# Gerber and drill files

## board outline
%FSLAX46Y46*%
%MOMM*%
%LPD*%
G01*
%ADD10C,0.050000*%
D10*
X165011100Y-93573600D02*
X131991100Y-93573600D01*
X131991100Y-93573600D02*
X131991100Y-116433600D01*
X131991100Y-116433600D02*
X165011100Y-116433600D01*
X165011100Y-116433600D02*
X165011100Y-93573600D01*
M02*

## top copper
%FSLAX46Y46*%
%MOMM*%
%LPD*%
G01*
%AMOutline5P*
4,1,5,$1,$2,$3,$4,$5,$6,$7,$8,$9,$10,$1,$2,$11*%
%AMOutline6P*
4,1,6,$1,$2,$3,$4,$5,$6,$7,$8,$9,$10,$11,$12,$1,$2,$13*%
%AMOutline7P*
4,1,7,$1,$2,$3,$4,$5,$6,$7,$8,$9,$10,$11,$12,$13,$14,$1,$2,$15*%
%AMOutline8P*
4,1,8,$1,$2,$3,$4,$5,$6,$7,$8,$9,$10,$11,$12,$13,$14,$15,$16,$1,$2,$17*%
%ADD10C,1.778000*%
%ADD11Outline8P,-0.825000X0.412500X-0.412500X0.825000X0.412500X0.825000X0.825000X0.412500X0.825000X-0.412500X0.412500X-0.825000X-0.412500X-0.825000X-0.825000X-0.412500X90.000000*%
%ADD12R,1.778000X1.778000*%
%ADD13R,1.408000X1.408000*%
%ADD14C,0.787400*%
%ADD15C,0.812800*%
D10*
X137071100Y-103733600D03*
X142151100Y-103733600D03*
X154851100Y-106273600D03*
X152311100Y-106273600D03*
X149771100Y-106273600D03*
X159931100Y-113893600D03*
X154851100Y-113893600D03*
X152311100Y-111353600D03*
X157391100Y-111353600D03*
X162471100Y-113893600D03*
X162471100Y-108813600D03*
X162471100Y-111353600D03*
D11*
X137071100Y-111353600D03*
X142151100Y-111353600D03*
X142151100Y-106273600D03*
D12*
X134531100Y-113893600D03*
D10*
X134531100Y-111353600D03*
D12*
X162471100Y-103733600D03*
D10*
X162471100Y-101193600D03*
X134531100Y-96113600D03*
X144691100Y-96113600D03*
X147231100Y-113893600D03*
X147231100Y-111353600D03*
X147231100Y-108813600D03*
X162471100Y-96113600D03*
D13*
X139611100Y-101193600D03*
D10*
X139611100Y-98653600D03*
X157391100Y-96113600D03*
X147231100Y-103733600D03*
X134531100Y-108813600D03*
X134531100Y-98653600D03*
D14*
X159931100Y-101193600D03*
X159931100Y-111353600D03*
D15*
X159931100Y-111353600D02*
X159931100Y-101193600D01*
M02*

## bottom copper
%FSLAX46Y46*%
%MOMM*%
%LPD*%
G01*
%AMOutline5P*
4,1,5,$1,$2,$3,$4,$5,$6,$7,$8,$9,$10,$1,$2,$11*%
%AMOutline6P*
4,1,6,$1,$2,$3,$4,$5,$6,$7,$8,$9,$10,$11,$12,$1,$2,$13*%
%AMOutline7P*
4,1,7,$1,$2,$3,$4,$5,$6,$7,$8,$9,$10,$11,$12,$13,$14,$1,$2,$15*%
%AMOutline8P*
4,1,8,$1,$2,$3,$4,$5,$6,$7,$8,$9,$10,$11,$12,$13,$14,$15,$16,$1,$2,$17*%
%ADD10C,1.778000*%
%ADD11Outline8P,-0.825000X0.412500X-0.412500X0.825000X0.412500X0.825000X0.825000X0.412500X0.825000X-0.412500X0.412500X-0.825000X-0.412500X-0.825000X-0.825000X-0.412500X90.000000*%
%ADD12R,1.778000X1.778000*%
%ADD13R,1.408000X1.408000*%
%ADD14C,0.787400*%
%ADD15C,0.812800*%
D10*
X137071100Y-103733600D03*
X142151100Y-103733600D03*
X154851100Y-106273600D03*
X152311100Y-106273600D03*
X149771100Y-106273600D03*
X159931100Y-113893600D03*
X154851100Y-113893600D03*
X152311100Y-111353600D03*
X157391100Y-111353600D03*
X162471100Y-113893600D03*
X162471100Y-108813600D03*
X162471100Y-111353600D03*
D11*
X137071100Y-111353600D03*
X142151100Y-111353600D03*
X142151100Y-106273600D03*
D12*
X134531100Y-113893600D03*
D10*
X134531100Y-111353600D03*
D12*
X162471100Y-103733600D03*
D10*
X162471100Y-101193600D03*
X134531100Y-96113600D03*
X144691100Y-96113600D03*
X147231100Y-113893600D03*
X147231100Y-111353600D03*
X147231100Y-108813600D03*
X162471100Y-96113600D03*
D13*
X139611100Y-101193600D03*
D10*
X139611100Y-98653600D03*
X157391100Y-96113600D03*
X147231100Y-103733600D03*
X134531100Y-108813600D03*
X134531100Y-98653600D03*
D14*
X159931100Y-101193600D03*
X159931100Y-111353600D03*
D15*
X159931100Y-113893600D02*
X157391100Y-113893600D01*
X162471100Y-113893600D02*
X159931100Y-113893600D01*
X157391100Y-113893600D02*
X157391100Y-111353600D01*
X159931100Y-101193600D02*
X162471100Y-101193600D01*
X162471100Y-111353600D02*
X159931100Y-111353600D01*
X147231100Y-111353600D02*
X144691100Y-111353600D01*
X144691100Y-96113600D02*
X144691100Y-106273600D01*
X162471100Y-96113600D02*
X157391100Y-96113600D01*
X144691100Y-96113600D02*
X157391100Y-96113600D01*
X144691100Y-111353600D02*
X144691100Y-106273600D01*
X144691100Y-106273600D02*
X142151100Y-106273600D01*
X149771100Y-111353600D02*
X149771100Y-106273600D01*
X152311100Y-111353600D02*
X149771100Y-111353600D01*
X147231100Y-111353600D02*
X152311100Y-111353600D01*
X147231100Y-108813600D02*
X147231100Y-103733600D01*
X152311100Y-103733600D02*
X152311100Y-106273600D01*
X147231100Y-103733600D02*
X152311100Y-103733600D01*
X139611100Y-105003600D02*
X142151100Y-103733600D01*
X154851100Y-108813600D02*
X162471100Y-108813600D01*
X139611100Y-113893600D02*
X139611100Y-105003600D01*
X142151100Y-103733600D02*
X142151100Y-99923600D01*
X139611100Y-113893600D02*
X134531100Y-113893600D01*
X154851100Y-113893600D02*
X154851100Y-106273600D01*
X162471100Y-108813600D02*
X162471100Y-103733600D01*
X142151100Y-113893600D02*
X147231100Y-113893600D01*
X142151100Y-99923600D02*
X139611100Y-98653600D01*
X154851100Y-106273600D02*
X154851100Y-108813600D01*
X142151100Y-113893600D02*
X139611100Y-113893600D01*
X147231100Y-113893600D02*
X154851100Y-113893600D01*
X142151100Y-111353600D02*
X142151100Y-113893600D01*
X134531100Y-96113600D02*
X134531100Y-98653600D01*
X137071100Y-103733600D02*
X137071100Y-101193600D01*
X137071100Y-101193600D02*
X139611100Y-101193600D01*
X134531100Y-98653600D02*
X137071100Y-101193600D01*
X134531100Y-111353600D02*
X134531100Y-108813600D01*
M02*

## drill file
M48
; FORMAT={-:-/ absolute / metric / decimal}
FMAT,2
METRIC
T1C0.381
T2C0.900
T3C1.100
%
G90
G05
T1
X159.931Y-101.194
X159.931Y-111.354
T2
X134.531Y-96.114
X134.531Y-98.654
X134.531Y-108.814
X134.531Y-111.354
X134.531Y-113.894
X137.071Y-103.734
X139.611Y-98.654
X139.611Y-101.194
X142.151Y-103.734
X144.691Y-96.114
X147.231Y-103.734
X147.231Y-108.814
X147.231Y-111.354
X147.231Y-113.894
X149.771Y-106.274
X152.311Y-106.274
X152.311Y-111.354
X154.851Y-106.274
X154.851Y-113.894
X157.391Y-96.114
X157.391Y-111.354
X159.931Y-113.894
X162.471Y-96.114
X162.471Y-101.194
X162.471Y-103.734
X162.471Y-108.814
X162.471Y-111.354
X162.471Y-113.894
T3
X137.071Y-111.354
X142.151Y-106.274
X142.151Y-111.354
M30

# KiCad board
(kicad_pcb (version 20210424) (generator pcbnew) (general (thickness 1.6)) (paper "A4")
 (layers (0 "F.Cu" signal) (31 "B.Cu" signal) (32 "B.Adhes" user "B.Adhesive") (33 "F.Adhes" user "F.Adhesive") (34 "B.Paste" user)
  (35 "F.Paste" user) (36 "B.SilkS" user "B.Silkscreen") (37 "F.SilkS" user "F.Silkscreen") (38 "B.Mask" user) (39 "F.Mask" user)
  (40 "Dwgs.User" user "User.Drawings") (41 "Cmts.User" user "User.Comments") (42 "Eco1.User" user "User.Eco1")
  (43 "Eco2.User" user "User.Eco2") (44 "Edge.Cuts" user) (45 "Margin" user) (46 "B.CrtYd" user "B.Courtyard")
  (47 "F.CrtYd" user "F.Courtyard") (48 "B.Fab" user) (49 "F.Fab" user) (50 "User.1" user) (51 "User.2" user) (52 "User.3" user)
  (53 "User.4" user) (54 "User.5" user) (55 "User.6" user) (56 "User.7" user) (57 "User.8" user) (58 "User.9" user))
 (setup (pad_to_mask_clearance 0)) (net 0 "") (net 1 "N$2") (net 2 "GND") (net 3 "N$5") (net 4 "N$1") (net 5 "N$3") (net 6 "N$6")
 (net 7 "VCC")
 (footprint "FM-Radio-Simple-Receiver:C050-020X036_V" (layer "F.Cu") (at 139.6111 103.7336 -90)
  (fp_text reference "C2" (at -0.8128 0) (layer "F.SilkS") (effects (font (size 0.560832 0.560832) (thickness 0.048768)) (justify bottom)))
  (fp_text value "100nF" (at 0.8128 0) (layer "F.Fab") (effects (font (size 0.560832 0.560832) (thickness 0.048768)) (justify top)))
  (pad "1" thru_hole circle (at 0 2.54 270) (size 1.778 1.778) (drill 0.9) (layers *.Cu *.Mask) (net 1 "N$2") (solder_mask_margin 0.1016))
  (pad "2" thru_hole circle (at 0 -2.54 270) (size 1.778 1.778) (drill 0.9) (layers *.Cu *.Mask) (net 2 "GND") (solder_mask_margin 0.1016)))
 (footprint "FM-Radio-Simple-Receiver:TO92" (layer "F.Cu") (at 152.3111 106.2736 -90)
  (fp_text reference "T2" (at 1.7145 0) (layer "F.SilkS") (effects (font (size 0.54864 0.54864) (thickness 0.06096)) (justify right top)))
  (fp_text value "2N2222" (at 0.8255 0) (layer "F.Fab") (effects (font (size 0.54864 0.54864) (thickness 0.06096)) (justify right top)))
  (pad "1" thru_hole circle (at 0 -2.54 180) (size 1.778 1.778) (drill 0.9) (layers *.Cu *.Mask) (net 2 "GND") (solder_mask_margin 0.1016))
  (pad "2" thru_hole circle (at 0 0 180) (size 1.778 1.778) (drill 0.9) (layers *.Cu *.Mask) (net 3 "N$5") (solder_mask_margin 0.1016))
  (pad "3" thru_hole circle (at 0 2.54 180) (size 1.778 1.778) (drill 0.9) (layers *.Cu *.Mask) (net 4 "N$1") (solder_mask_margin 0.1016)))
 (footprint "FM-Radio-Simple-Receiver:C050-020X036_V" (layer "F.Cu") (at 157.3911 113.8936 90)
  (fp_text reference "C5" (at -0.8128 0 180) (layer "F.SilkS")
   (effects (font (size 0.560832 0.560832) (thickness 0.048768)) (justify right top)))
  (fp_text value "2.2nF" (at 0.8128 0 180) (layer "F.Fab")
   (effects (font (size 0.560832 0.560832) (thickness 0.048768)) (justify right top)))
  (pad "1" thru_hole circle (at 0 2.54 90) (size 1.778 1.778) (drill 0.9) (layers *.Cu *.Mask) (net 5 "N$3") (solder_mask_margin 0.1016))
  (pad "2" thru_hole circle (at 0 -2.54 90) (size 1.778 1.778) (drill 0.9) (layers *.Cu *.Mask) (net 2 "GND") (solder_mask_margin 0.1016)))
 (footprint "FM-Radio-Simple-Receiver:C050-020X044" (layer "F.Cu") (at 154.8511 111.3536)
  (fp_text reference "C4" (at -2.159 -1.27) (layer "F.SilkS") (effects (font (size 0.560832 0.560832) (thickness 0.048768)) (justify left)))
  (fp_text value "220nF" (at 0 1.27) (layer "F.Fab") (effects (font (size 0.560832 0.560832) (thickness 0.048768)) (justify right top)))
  (pad "1" thru_hole circle (at -2.54 0) (size 1.778 1.778) (drill 0.9) (layers *.Cu *.Mask) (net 4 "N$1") (solder_mask_margin 0.1016))
  (pad "2" thru_hole circle (at 2.54 0) (size 1.778 1.778) (drill 0.9) (layers *.Cu *.Mask) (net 5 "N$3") (solder_mask_margin 0.1016)))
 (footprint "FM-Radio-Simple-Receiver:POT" (layer "F.Cu") (at 162.4711 111.3536 90)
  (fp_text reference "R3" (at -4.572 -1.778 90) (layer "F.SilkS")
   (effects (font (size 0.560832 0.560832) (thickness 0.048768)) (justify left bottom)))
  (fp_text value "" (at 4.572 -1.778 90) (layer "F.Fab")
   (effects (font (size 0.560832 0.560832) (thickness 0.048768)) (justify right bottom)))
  (pad "A" thru_hole circle (at -2.54 0 90) (size 1.778 1.778) (drill 0.9) (layers *.Cu *.Mask) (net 5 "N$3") (solder_mask_margin 0.1016))
  (pad "E" thru_hole circle (at 2.54 0 90) (size 1.778 1.778) (drill 0.9) (layers *.Cu *.Mask) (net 2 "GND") (solder_mask_margin 0.1016))
  (pad "S" thru_hole circle (at 0 0 90) (size 1.778 1.778) (drill 0.9) (layers *.Cu *.Mask) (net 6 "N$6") (solder_mask_margin 0.1016)))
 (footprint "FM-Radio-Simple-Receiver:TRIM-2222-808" (layer "F.Cu") (at 139.6111 108.8136 90)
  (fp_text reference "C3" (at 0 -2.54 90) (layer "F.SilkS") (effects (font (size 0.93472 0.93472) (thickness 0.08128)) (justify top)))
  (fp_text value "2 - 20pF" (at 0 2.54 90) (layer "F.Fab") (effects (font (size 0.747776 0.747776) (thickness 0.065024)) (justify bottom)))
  (pad "1" thru_hole roundrect (at -2.54 -2.54 90) (size 1.65 1.65) (drill 1.1) (layers *.Cu *.Mask) (roundrect_rratio 0.25)
   (chamfer_ratio 0.25) (chamfer top_left top_right bottom_left bottom_right) (solder_mask_margin 0.1016))
  (pad "2" thru_hole roundrect (at -2.54 2.54 90) (size 1.65 1.65) (drill 1.1) (layers *.Cu *.Mask) (roundrect_rratio 0.25)
   (chamfer_ratio 0.25) (chamfer top_left top_right bottom_left bottom_right) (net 2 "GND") (solder_mask_margin 0.1016))
  (pad "3" thru_hole roundrect (at 2.54 2.54 90) (size 1.65 1.65) (drill 1.1) (layers *.Cu *.Mask) (roundrect_rratio 0.25)
   (chamfer_ratio 0.25) (chamfer top_left top_right bottom_left bottom_right) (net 4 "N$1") (solder_mask_margin 0.1016)))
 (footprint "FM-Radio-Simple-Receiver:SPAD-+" (layer "F.Cu") (at 134.5311 112.6236)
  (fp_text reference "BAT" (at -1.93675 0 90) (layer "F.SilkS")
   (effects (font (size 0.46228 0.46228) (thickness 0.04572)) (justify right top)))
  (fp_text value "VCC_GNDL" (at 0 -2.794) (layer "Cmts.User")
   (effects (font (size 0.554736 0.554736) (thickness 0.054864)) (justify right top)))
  (pad "1" thru_hole rect (at 0 1.27 180) (size 1.778 1.778) (drill 0.9) (layers *.Cu) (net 2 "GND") (solder_mask_margin 0.1016))
  (pad "2" thru_hole circle (at 0 -1.27) (size 1.778 1.778) (drill 0.9) (layers *.Cu) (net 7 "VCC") (solder_mask_margin 0.1016)))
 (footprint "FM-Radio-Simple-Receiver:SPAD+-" (layer "F.Cu") (at 162.4711 102.4636)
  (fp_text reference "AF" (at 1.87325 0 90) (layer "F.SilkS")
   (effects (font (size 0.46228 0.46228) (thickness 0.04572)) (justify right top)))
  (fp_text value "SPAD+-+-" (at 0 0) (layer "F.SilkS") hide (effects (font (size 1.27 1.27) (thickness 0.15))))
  (pad "1" thru_hole rect (at 0 1.27) (size 1.778 1.778) (drill 0.9) (layers *.Cu) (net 2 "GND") (solder_mask_margin 0.1016))
  (pad "2" thru_hole circle (at 0 -1.27) (size 1.778 1.778) (drill 0.9) (layers *.Cu) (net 6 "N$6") (solder_mask_margin 0.1016)))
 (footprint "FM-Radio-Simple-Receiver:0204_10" (layer "F.Cu") (at 139.6111 96.1136)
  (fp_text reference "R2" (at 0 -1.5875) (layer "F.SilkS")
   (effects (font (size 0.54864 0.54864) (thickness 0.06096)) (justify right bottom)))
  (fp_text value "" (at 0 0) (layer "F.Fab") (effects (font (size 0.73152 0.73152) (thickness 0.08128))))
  (pad "1" thru_hole circle (at -5.08 0) (size 1.778 1.778) (drill 0.9) (layers *.Cu *.Mask) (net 1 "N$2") (solder_mask_margin 0.1016))
  (pad "2" thru_hole circle (at 5.08 0) (size 1.778 1.778) (drill 0.9) (layers *.Cu *.Mask) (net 4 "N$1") (solder_mask_margin 0.1016)))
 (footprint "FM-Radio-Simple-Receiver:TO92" (layer "F.Cu") (at 147.2311 111.3536 180)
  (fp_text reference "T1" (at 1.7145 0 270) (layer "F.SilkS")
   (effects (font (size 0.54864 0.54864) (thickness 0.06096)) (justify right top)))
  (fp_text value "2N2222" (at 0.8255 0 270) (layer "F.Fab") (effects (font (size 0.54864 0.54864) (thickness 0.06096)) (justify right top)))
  (pad "1" thru_hole circle (at 0 -2.54 90) (size 1.778 1.778) (drill 0.9) (layers *.Cu *.Mask) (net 2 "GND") (solder_mask_margin 0.1016))
  (pad "2" thru_hole circle (at 0 0 90) (size 1.778 1.778) (drill 0.9) (layers *.Cu *.Mask) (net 4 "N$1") (solder_mask_margin 0.1016))
  (pad "3" thru_hole circle (at 0 2.54 90) (size 1.778 1.778) (drill 0.9) (layers *.Cu *.Mask) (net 3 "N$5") (solder_mask_margin 0.1016)))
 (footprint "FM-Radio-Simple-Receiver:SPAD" (layer "F.Cu") (at 162.4711 96.1136 -90)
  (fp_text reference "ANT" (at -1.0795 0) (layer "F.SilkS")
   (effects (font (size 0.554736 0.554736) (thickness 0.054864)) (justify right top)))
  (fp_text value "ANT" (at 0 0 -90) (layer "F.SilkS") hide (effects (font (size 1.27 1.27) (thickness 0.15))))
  (pad "1" thru_hole circle (at 0 0 270) (size 1.778 1.778) (drill 0.9) (layers *.Cu) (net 4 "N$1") (solder_mask_margin 0.1016)))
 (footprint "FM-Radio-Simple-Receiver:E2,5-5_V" (layer "F.Cu") (at 139.6111 99.9236)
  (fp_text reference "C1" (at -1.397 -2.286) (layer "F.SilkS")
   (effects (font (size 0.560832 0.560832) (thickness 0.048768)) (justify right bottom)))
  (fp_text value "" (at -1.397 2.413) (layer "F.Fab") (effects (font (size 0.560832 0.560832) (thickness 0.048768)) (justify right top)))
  (pad "+" thru_hole rect (at 0 1.27) (size 1.408 1.408) (drill 0.9) (layers *.Cu *.Mask) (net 1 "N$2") (solder_mask_margin 0.1016))
  (pad "-" thru_hole circle (at 0 -1.27) (size 1.778 1.778) (drill 0.9) (layers *.Cu *.Mask) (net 2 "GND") (solder_mask_margin 0.1016)))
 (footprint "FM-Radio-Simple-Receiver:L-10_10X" (layer "F.Cu") (at 154.8511 101.1936 -90)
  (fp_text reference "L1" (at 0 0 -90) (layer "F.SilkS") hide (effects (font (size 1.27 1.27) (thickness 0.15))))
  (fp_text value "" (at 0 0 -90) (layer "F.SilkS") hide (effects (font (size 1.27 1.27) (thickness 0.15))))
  (pad "P$1" thru_hole circle (at -5.08 -2.54 270) (size 1.778 1.778) (drill 0.9) (layers *.Cu *.Mask) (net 4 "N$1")
   (solder_mask_margin 0.1016))
  (pad "P$2" thru_hole circle (at 2.54 7.62 270) (size 1.778 1.778) (drill 0.9) (layers *.Cu *.Mask) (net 3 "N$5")
   (solder_mask_margin 0.1016)))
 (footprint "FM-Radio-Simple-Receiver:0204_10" (layer "F.Cu") (at 134.5311 103.7336 90)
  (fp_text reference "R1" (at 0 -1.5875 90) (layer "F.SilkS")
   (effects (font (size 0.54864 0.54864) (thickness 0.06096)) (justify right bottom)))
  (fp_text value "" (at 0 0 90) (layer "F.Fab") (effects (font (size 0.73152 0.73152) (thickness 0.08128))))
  (pad "1" thru_hole circle (at -5.08 0 90) (size 1.778 1.778) (drill 0.9) (layers *.Cu *.Mask) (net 7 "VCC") (solder_mask_margin 0.1016))
  (pad "2" thru_hole circle (at 5.08 0 90) (size 1.778 1.778) (drill 0.9) (layers *.Cu *.Mask) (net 1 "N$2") (solder_mask_margin 0.1016)))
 (gr_line (start 165.0111 93.5736) (end 131.9911 93.5736) (layer "Edge.Cuts") (width 0.05))
 (gr_line (start 131.9911 93.5736) (end 131.9911 116.4336) (layer "Edge.Cuts") (width 0.05))
 (gr_line (start 131.9911 116.4336) (end 165.0111 116.4336) (layer "Edge.Cuts") (width 0.05))
 (gr_line (start 165.0111 116.4336) (end 165.0111 93.5736) (layer "Edge.Cuts") (width 0.05))
 (segment (start 159.9311 113.8936) (end 157.3911 113.8936) (width 0.8128) (layer "B.Cu") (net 5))
 (segment (start 162.4711 113.8936) (end 159.9311 113.8936) (width 0.8128) (layer "B.Cu") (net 5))
 (segment (start 157.3911 113.8936) (end 157.3911 111.3536) (width 0.8128) (layer "B.Cu") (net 5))
 (segment (start 159.9311 111.3536) (end 159.9311 101.1936) (width 0.8128) (layer "F.Cu") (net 6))
 (via (at 159.9311 101.1936) (size 0.7874) (drill 0.381) (layers "F.Cu" "B.Cu") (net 6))
 (via (at 159.9311 111.3536) (size 0.7874) (drill 0.381) (layers "F.Cu" "B.Cu") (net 6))
 (segment (start 159.9311 101.1936) (end 162.4711 101.1936) (width 0.8128) (layer "B.Cu") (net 6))
 (segment (start 162.4711 111.3536) (end 159.9311 111.3536) (width 0.8128) (layer "B.Cu") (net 6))
 (segment (start 147.2311 111.3536) (end 144.6911 111.3536) (width 0.8128) (layer "B.Cu") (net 4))
 (segment (start 144.6911 96.1136) (end 144.6911 106.2736) (width 0.8128) (layer "B.Cu") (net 4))
 (segment (start 162.4711 96.1136) (end 157.3911 96.1136) (width 0.8128) (layer "B.Cu") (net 4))
 (segment (start 144.6911 96.1136) (end 157.3911 96.1136) (width 0.8128) (layer "B.Cu") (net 4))
 (segment (start 144.6911 111.3536) (end 144.6911 106.2736) (width 0.8128) (layer "B.Cu") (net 4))
 (segment (start 144.6911 106.2736) (end 142.1511 106.2736) (width 0.8128) (layer "B.Cu") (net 4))
 (segment (start 149.7711 111.3536) (end 149.7711 106.2736) (width 0.8128) (layer "B.Cu") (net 4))
 (segment (start 152.3111 111.3536) (end 149.7711 111.3536) (width 0.8128) (layer "B.Cu") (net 4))
 (segment (start 147.2311 111.3536) (end 152.3111 111.3536) (width 0.8128) (layer "B.Cu") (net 4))
 (segment (start 147.2311 108.8136) (end 147.2311 103.7336) (width 0.8128) (layer "B.Cu") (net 3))
 (segment (start 152.3111 103.7336) (end 152.3111 106.2736) (width 0.8128) (layer "B.Cu") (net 3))
 (segment (start 147.2311 103.7336) (end 152.3111 103.7336) (width 0.8128) (layer "B.Cu") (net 3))
 (segment (start 139.6111 105.0036) (end 142.1511 103.7336) (width 0.8128) (layer "B.Cu") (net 2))
 (segment (start 154.8511 108.8136) (end 162.4711 108.8136) (width 0.8128) (layer "B.Cu") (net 2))
 (segment (start 139.6111 113.8936) (end 139.6111 105.0036) (width 0.8128) (layer "B.Cu") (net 2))
 (segment (start 142.1511 103.7336) (end 142.1511 99.9236) (width 0.8128) (layer "B.Cu") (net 2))
 (segment (start 139.6111 113.8936) (end 134.5311 113.8936) (width 0.8128) (layer "B.Cu") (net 2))
 (segment (start 154.8511 113.8936) (end 154.8511 106.2736) (width 0.8128) (layer "B.Cu") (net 2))
 (segment (start 162.4711 108.8136) (end 162.4711 103.7336) (width 0.8128) (layer "B.Cu") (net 2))
 (segment (start 142.1511 113.8936) (end 147.2311 113.8936) (width 0.8128) (layer "B.Cu") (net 2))
 (segment (start 142.1511 99.9236) (end 139.6111 98.6536) (width 0.8128) (layer "B.Cu") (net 2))
 (segment (start 154.8511 106.2736) (end 154.8511 108.8136) (width 0.8128) (layer "B.Cu") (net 2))
 (segment (start 142.1511 113.8936) (end 139.6111 113.8936) (width 0.8128) (layer "B.Cu") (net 2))
 (segment (start 147.2311 113.8936) (end 154.8511 113.8936) (width 0.8128) (layer "B.Cu") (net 2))
 (segment (start 142.1511 111.3536) (end 142.1511 113.8936) (width 0.8128) (layer "B.Cu") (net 2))
 (segment (start 134.5311 96.1136) (end 134.5311 98.6536) (width 0.8128) (layer "B.Cu") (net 1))
 (segment (start 137.0711 103.7336) (end 137.0711 101.1936) (width 0.8128) (layer "B.Cu") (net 1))
 (segment (start 137.0711 101.1936) (end 139.6111 101.1936) (width 0.8128) (layer "B.Cu") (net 1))
 (segment (start 134.5311 98.6536) (end 137.0711 101.1936) (width 0.8128) (layer "B.Cu") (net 1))
 (segment (start 134.5311 111.3536) (end 134.5311 108.8136) (width 0.8128) (layer "B.Cu") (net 7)))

